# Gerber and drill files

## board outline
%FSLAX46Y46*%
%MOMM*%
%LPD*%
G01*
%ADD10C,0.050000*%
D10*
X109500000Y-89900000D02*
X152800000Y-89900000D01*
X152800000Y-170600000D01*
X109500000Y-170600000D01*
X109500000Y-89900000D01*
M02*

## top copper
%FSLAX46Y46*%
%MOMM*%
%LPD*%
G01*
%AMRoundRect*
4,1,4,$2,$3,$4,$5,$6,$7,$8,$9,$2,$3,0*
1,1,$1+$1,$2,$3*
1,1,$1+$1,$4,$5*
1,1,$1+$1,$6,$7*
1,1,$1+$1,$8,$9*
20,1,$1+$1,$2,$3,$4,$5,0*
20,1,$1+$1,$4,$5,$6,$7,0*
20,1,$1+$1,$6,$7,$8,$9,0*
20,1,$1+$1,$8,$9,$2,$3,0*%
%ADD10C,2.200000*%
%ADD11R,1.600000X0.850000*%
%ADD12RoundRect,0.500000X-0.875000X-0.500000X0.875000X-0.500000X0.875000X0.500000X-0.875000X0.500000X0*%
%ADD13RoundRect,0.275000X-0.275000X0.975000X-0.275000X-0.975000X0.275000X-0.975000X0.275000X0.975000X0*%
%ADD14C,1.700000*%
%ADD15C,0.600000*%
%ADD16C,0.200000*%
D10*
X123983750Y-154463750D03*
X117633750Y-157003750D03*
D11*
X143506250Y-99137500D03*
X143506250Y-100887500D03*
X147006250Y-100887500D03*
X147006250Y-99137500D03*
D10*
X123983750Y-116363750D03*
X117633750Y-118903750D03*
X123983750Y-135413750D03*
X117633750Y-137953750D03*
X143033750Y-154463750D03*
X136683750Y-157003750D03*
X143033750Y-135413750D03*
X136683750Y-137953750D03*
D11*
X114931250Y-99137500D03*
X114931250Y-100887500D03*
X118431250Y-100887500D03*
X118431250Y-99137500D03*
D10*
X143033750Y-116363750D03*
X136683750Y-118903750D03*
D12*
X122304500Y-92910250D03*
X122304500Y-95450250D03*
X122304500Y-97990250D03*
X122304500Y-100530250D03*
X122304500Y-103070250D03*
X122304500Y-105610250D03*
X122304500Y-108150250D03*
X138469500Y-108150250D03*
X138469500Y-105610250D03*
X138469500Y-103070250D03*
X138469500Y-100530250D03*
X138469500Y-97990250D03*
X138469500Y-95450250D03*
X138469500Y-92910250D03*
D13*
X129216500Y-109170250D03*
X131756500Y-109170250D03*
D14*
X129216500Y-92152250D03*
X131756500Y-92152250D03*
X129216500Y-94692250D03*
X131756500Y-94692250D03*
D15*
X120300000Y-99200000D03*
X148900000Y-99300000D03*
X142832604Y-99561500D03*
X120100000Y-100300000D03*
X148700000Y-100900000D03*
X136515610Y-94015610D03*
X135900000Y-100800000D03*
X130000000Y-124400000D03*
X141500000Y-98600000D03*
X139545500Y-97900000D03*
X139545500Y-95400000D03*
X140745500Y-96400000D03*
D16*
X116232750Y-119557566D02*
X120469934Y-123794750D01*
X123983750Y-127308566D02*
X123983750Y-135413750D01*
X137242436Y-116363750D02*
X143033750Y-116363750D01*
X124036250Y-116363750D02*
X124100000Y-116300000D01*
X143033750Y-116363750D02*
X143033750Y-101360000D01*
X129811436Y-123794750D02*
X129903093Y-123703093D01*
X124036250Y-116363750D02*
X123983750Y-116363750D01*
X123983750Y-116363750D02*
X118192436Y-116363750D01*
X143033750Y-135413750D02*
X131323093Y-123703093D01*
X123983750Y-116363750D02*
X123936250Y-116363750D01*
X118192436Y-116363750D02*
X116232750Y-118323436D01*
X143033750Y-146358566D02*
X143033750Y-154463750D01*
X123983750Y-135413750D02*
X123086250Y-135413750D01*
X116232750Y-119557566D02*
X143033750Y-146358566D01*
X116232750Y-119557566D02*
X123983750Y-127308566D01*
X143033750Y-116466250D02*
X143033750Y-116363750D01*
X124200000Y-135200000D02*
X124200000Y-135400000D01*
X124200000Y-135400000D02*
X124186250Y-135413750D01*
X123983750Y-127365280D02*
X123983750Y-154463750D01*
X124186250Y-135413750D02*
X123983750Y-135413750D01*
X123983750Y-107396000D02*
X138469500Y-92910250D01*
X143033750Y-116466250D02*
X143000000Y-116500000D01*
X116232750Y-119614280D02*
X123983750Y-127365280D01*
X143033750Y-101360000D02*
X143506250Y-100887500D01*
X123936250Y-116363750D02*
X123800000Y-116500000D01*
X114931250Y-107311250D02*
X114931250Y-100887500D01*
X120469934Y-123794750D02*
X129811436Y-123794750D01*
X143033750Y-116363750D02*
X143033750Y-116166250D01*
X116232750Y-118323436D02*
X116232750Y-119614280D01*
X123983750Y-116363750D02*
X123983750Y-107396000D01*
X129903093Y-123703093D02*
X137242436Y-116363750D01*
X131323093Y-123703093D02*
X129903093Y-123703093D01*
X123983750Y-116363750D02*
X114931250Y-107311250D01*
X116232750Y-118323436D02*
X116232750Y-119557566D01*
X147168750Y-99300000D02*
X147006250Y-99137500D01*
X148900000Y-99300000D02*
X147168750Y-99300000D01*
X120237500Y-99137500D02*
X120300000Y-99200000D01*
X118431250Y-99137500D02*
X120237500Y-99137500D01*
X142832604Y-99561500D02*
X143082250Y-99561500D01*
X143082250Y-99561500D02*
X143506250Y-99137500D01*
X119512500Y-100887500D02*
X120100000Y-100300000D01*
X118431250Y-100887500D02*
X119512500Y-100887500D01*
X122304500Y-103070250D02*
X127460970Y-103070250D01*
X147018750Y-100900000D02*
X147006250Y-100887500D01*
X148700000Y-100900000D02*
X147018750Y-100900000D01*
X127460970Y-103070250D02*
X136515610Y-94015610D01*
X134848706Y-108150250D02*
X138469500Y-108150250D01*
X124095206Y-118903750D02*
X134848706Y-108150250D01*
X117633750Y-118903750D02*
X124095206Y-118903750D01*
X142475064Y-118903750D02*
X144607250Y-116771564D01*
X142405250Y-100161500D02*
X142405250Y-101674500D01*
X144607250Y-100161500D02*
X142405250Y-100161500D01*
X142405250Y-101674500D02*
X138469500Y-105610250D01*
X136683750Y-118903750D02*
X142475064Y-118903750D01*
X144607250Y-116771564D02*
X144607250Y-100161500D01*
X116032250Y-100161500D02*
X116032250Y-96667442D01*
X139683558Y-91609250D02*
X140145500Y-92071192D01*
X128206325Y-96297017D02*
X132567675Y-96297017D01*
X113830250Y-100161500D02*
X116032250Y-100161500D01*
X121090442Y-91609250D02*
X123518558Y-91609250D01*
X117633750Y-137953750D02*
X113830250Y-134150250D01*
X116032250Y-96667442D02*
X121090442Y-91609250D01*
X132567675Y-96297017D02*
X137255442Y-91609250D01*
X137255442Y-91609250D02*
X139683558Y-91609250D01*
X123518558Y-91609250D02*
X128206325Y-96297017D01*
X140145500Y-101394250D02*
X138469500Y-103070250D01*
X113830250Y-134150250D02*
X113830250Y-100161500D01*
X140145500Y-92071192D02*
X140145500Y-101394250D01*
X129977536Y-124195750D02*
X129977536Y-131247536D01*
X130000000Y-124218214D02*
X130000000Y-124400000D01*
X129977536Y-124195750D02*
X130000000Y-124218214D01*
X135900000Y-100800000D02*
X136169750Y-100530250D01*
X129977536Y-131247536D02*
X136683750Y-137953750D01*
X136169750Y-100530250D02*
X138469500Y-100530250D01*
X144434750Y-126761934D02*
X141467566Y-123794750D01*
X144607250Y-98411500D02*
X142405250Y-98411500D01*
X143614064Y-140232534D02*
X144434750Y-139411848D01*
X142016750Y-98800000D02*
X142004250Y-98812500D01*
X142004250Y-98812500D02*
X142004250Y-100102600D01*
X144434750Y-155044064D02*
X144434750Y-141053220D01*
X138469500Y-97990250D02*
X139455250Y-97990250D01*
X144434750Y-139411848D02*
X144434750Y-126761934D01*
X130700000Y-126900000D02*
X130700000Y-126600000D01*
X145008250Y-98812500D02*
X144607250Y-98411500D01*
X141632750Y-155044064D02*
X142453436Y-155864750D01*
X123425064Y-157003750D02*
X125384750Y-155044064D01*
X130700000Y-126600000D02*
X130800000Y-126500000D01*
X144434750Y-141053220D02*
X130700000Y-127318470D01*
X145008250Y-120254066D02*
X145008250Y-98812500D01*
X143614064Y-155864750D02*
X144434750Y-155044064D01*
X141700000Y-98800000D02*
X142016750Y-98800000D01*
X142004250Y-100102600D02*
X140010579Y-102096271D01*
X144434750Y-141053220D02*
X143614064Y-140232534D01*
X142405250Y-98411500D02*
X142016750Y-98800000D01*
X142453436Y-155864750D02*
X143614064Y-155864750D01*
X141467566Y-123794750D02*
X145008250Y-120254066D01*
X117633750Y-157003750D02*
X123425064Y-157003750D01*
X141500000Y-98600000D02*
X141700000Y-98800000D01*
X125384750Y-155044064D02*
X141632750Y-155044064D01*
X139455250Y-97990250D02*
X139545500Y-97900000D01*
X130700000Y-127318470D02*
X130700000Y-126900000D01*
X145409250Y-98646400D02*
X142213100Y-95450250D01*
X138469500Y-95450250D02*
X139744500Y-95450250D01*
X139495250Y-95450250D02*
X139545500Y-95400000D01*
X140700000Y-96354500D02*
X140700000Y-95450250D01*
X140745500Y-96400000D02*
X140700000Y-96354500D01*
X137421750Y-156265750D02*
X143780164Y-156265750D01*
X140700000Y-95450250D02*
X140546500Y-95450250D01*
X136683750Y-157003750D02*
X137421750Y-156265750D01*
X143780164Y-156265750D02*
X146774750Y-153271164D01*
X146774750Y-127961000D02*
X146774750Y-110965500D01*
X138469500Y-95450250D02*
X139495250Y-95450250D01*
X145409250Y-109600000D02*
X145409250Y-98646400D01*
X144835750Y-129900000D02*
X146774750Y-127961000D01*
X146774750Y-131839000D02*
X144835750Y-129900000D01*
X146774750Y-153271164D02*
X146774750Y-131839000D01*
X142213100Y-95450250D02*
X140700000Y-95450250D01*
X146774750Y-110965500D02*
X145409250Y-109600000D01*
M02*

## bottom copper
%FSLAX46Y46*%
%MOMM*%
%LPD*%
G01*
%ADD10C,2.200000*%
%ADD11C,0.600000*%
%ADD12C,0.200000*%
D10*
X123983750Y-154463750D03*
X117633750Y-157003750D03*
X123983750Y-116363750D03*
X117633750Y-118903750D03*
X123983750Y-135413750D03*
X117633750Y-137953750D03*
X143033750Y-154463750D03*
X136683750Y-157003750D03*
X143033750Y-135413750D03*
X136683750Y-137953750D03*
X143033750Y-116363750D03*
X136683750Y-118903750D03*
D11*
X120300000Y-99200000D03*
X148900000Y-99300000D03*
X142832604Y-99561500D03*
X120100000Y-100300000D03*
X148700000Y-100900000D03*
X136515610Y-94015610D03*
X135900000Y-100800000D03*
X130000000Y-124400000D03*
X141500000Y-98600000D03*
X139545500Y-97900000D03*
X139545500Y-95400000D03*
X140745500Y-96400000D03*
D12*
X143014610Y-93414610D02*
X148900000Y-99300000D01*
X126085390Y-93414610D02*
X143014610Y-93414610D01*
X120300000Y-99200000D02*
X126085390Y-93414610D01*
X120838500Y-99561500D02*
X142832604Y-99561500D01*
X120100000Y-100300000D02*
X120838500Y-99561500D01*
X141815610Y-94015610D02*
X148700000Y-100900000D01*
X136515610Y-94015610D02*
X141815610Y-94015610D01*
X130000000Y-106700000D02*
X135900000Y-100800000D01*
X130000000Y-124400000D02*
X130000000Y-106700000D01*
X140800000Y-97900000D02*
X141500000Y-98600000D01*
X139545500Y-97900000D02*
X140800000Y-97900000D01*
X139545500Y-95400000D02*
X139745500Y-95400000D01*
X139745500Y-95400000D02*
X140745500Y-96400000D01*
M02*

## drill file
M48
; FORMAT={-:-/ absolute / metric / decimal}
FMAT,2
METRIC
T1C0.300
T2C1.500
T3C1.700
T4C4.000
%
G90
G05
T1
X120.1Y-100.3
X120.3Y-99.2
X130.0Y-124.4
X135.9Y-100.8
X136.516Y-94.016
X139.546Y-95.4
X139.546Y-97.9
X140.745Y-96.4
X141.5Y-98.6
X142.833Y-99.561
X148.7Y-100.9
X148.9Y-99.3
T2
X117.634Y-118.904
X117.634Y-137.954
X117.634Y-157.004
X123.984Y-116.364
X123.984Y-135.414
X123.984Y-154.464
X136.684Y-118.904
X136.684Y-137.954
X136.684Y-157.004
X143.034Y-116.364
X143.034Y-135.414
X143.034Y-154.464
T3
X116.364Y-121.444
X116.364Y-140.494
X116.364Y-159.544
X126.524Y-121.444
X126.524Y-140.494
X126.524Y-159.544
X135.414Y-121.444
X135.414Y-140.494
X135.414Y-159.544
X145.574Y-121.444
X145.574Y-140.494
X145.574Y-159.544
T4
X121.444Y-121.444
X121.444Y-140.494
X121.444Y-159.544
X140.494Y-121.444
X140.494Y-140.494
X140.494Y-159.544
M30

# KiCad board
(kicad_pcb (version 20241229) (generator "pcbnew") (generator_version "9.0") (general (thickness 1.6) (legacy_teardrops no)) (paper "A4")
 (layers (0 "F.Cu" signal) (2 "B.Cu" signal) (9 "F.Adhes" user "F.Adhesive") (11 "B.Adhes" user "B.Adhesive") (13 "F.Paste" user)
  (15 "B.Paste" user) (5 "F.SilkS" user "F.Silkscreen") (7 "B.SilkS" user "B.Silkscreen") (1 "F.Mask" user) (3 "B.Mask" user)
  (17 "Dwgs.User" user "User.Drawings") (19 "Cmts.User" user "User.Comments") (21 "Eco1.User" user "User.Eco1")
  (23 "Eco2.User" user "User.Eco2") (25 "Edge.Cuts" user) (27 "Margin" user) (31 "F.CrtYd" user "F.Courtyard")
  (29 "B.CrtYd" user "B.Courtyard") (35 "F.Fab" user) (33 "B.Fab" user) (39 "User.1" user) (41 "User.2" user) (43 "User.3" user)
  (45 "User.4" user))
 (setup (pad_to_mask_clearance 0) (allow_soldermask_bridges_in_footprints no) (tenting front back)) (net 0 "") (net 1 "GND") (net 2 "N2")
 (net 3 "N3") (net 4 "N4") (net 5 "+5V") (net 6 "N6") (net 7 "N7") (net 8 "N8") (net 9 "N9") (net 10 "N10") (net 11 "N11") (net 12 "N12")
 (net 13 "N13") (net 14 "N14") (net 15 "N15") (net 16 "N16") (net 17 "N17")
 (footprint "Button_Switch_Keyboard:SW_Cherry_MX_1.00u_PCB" (layer "F.Cu") (at 123.98375 154.46375)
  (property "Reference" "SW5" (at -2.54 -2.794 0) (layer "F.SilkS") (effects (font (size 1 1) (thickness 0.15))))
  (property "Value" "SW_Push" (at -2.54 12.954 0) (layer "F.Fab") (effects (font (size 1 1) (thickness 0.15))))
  (pad "" np_thru_hole circle (at -7.62 5.08) (size 1.7 1.7) (drill 1.7) (layers "*.Cu" "*.Mask"))
  (pad "" np_thru_hole circle (at -2.54 5.08) (size 4 4) (drill 4) (layers "*.Cu" "*.Mask"))
  (pad "" np_thru_hole circle (at 2.54 5.08) (size 1.7 1.7) (drill 1.7) (layers "*.Cu" "*.Mask"))
  (pad "1" thru_hole circle (at 0 0) (size 2.2 2.2) (drill 1.5) (layers "*.Cu" "*.Mask") (remove_unused_layers no) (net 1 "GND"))
  (pad "2" thru_hole circle (at -6.35 2.54) (size 2.2 2.2) (drill 1.5) (layers "*.Cu" "*.Mask") (remove_unused_layers no) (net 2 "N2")))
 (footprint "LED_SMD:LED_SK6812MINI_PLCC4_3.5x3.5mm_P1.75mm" (layer "F.Cu") (at 145.25625 100.0125)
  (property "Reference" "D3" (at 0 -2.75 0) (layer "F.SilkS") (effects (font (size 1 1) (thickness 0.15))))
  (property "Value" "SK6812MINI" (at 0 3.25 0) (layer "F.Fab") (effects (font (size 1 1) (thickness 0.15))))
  (pad "1" smd rect (at -1.75 -0.875) (size 1.6 0.85) (layers "F.Cu" "F.Mask" "F.Paste") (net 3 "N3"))
  (pad "2" smd rect (at -1.75 0.875) (size 1.6 0.85) (layers "F.Cu" "F.Mask" "F.Paste") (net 1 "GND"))
  (pad "3" smd rect (at 1.75 0.875) (size 1.6 0.85) (layers "F.Cu" "F.Mask" "F.Paste") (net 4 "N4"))
  (pad "4" smd rect (at 1.75 -0.875) (size 1.6 0.85) (layers "F.Cu" "F.Mask" "F.Paste") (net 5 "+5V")))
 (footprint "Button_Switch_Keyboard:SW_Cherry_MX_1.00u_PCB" (layer "F.Cu") (at 123.98375 116.36375)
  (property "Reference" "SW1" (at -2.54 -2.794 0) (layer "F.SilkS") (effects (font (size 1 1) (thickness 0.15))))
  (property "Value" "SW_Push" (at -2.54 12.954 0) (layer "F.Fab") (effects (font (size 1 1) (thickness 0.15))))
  (pad "" np_thru_hole circle (at -7.62 5.08) (size 1.7 1.7) (drill 1.7) (layers "*.Cu" "*.Mask"))
  (pad "" np_thru_hole circle (at -2.54 5.08) (size 4 4) (drill 4) (layers "*.Cu" "*.Mask"))
  (pad "" np_thru_hole circle (at 2.54 5.08) (size 1.7 1.7) (drill 1.7) (layers "*.Cu" "*.Mask"))
  (pad "1" thru_hole circle (at 0 0) (size 2.2 2.2) (drill 1.5) (layers "*.Cu" "*.Mask") (remove_unused_layers no) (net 1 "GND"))
  (pad "2" thru_hole circle (at -6.35 2.54) (size 2.2 2.2) (drill 1.5) (layers "*.Cu" "*.Mask") (remove_unused_layers no) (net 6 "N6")))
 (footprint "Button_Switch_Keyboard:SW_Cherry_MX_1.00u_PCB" (layer "F.Cu") (at 123.98375 135.41375)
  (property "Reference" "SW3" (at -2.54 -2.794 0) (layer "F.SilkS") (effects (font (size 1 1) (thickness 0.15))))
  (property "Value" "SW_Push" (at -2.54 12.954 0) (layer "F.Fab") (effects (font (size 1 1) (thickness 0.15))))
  (pad "" np_thru_hole circle (at -7.62 5.08) (size 1.7 1.7) (drill 1.7) (layers "*.Cu" "*.Mask"))
  (pad "" np_thru_hole circle (at -2.54 5.08) (size 4 4) (drill 4) (layers "*.Cu" "*.Mask"))
  (pad "" np_thru_hole circle (at 2.54 5.08) (size 1.7 1.7) (drill 1.7) (layers "*.Cu" "*.Mask"))
  (pad "1" thru_hole circle (at 0 0) (size 2.2 2.2) (drill 1.5) (layers "*.Cu" "*.Mask") (remove_unused_layers no) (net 1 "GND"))
  (pad "2" thru_hole circle (at -6.35 2.54) (size 2.2 2.2) (drill 1.5) (layers "*.Cu" "*.Mask") (remove_unused_layers no) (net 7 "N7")))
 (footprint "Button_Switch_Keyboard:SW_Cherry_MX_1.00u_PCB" (layer "F.Cu") (at 143.03375 154.46375)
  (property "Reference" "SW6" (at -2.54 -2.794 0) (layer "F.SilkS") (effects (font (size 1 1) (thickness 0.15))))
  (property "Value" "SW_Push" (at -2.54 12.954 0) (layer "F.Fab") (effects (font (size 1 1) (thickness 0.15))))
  (pad "" np_thru_hole circle (at -7.62 5.08) (size 1.7 1.7) (drill 1.7) (layers "*.Cu" "*.Mask"))
  (pad "" np_thru_hole circle (at -2.54 5.08) (size 4 4) (drill 4) (layers "*.Cu" "*.Mask"))
  (pad "" np_thru_hole circle (at 2.54 5.08) (size 1.7 1.7) (drill 1.7) (layers "*.Cu" "*.Mask"))
  (pad "1" thru_hole circle (at 0 0) (size 2.2 2.2) (drill 1.5) (layers "*.Cu" "*.Mask") (remove_unused_layers no) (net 1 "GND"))
  (pad "2" thru_hole circle (at -6.35 2.54) (size 2.2 2.2) (drill 1.5) (layers "*.Cu" "*.Mask") (remove_unused_layers no) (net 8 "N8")))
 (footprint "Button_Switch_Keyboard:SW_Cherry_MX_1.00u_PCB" (layer "F.Cu") (at 143.03375 135.41375)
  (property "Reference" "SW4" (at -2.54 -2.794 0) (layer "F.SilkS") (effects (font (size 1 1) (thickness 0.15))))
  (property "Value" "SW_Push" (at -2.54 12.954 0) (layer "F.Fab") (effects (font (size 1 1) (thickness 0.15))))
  (pad "" np_thru_hole circle (at -7.62 5.08) (size 1.7 1.7) (drill 1.7) (layers "*.Cu" "*.Mask"))
  (pad "" np_thru_hole circle (at -2.54 5.08) (size 4 4) (drill 4) (layers "*.Cu" "*.Mask"))
  (pad "" np_thru_hole circle (at 2.54 5.08) (size 1.7 1.7) (drill 1.7) (layers "*.Cu" "*.Mask"))
  (pad "1" thru_hole circle (at 0 0) (size 2.2 2.2) (drill 1.5) (layers "*.Cu" "*.Mask") (remove_unused_layers no) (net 1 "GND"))
  (pad "2" thru_hole circle (at -6.35 2.54) (size 2.2 2.2) (drill 1.5) (layers "*.Cu" "*.Mask") (remove_unused_layers no) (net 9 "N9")))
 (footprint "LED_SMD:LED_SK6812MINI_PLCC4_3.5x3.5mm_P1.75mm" (layer "F.Cu") (at 116.68125 100.0125)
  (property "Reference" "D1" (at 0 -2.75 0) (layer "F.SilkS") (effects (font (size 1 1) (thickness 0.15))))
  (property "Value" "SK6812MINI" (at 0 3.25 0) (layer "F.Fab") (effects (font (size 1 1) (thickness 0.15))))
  (pad "1" smd rect (at -1.75 -0.875) (size 1.6 0.85) (layers "F.Cu" "F.Mask" "F.Paste") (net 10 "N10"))
  (pad "2" smd rect (at -1.75 0.875) (size 1.6 0.85) (layers "F.Cu" "F.Mask" "F.Paste") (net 1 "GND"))
  (pad "3" smd rect (at 1.75 0.875) (size 1.6 0.85) (layers "F.Cu" "F.Mask" "F.Paste") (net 3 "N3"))
  (pad "4" smd rect (at 1.75 -0.875) (size 1.6 0.85) (layers "F.Cu" "F.Mask" "F.Paste") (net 5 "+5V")))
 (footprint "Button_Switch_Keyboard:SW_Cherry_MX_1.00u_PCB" (layer "F.Cu") (at 143.03375 116.36375)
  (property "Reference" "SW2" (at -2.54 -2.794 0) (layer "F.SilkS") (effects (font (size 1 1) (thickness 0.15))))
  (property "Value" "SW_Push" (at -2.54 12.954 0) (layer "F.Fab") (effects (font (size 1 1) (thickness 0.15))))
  (pad "" np_thru_hole circle (at -7.62 5.08) (size 1.7 1.7) (drill 1.7) (layers "*.Cu" "*.Mask"))
  (pad "" np_thru_hole circle (at -2.54 5.08) (size 4 4) (drill 4) (layers "*.Cu" "*.Mask"))
  (pad "" np_thru_hole circle (at 2.54 5.08) (size 1.7 1.7) (drill 1.7) (layers "*.Cu" "*.Mask"))
  (pad "1" thru_hole circle (at 0 0) (size 2.2 2.2) (drill 1.5) (layers "*.Cu" "*.Mask") (remove_unused_layers no) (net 1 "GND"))
  (pad "2" thru_hole circle (at -6.35 2.54) (size 2.2 2.2) (drill 1.5) (layers "*.Cu" "*.Mask") (remove_unused_layers no) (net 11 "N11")))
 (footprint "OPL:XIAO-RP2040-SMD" (layer "F.Cu") (at 130.3045 100.53025)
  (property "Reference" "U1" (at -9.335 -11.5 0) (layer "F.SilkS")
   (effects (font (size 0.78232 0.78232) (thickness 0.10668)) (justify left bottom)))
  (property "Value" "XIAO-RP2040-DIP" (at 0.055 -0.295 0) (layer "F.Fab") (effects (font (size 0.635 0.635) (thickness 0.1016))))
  (pad "1" smd roundrect (at -8 -7.62) (size 2.75 2) (layers "F.Cu" "F.Mask" "F.Paste") (roundrect_rratio 0.25) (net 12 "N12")
   (solder_mask_margin 0.0508) (thermal_bridge_angle 45))
  (pad "2" smd roundrect (at -8 -5.08) (size 2.75 2) (layers "F.Cu" "F.Mask" "F.Paste") (roundrect_rratio 0.25) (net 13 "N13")
   (solder_mask_margin 0.0508) (thermal_bridge_angle 45))
  (pad "3" smd roundrect (at -8 -2.54) (size 2.75 2) (layers "F.Cu" "F.Mask" "F.Paste") (roundrect_rratio 0.25) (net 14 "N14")
   (solder_mask_margin 0.0508) (thermal_bridge_angle 45))
  (pad "4" smd roundrect (at -8 0) (size 2.75 2) (layers "F.Cu" "F.Mask" "F.Paste") (roundrect_rratio 0.25) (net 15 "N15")
   (solder_mask_margin 0.0508) (thermal_bridge_angle 45))
  (pad "5" smd roundrect (at -8 2.54) (size 2.75 2) (layers "F.Cu" "F.Mask" "F.Paste") (roundrect_rratio 0.25) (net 4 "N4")
   (solder_mask_margin 0.0508) (thermal_bridge_angle 45))
  (pad "6" smd roundrect (at -8 5.08) (size 2.75 2) (layers "F.Cu" "F.Mask" "F.Paste") (roundrect_rratio 0.25) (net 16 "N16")
   (solder_mask_margin 0.0508) (thermal_bridge_angle 45))
  (pad "7" smd roundrect (at -8 7.62) (size 2.75 2) (layers "F.Cu" "F.Mask" "F.Paste") (roundrect_rratio 0.25) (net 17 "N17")
   (solder_mask_margin 0.0508) (thermal_bridge_angle 45))
  (pad "8" smd roundrect (at 8.165 7.62) (size 2.75 2) (layers "F.Cu" "F.Mask" "F.Paste") (roundrect_rratio 0.25) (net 6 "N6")
   (solder_mask_margin 0.0508) (thermal_bridge_angle 45))
  (pad "9" smd roundrect (at 8.165 5.08) (size 2.75 2) (layers "F.Cu" "F.Mask" "F.Paste") (roundrect_rratio 0.25) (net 11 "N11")
   (solder_mask_margin 0.0508) (thermal_bridge_angle 45))
  (pad "10" smd roundrect (at 8.165 2.54) (size 2.75 2) (layers "F.Cu" "F.Mask" "F.Paste") (roundrect_rratio 0.25) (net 7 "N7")
   (solder_mask_margin 0.0508) (thermal_bridge_angle 45))
  (pad "11" smd roundrect (at 8.165 0) (size 2.75 2) (layers "F.Cu" "F.Mask" "F.Paste") (roundrect_rratio 0.25) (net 9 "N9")
   (solder_mask_margin 0.0508) (thermal_bridge_angle 45))
  (pad "12" smd roundrect (at 8.165 -2.54) (size 2.75 2) (layers "F.Cu" "F.Mask" "F.Paste") (roundrect_rratio 0.25) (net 2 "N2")
   (solder_mask_margin 0.0508) (thermal_bridge_angle 45))
  (pad "13" smd roundrect (at 8.165 -5.08) (size 2.75 2) (layers "F.Cu" "F.Mask" "F.Paste") (roundrect_rratio 0.25) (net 8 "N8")
   (solder_mask_margin 0.0508) (thermal_bridge_angle 45))
  (pad "14" smd roundrect (at 8.165 -7.62) (size 2.75 2) (layers "F.Cu" "F.Mask" "F.Paste") (roundrect_rratio 0.25) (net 1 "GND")
   (solder_mask_margin 0.0508) (thermal_bridge_angle 45))
  (pad "15" smd roundrect (at -1.088 8.64 270) (size 2.5 1.1) (layers "F.Cu" "F.Mask" "F.Paste") (roundrect_rratio 0.25)
   (thermal_bridge_angle 45))
  (pad "16" smd roundrect (at 1.452 8.64 270) (size 2.5 1.1) (layers "F.Cu" "F.Mask" "F.Paste") (roundrect_rratio 0.25)
   (thermal_bridge_angle 45))
  (pad "17" smd circle (at -1.088 -8.378) (size 1.7 1.7) (layers "F.Cu" "F.Mask" "F.Paste"))
  (pad "18" smd circle (at 1.452 -8.378) (size 1.7 1.7) (layers "F.Cu" "F.Mask" "F.Paste"))
  (pad "19" smd circle (at -1.088 -5.838) (size 1.7 1.7) (layers "F.Cu" "F.Mask" "F.Paste"))
  (pad "20" smd circle (at 1.452 -5.838) (size 1.7 1.7) (layers "F.Cu" "F.Mask" "F.Paste")))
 (gr_rect (start 109.5 89.9) (end 152.8 170.6) (stroke (width 0.05) (type default)) (fill no) (layer "Edge.Cuts"))
 (segment (start 116.23275 119.557566) (end 120.469934 123.79475) (width 0.2) (layer "F.Cu") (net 1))
 (segment (start 123.98375 127.308566) (end 123.98375 135.41375) (width 0.2) (layer "F.Cu") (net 1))
 (segment (start 137.242436 116.36375) (end 143.03375 116.36375) (width 0.2) (layer "F.Cu") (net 1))
 (segment (start 124.03625 116.36375) (end 124.1 116.3) (width 0.2) (layer "F.Cu") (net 1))
 (segment (start 143.03375 116.36375) (end 143.03375 101.36) (width 0.2) (layer "F.Cu") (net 1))
 (segment (start 129.811436 123.79475) (end 129.903093 123.703093) (width 0.2) (layer "F.Cu") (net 1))
 (segment (start 124.03625 116.36375) (end 123.98375 116.36375) (width 0.2) (layer "F.Cu") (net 1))
 (segment (start 123.98375 116.36375) (end 118.192436 116.36375) (width 0.2) (layer "F.Cu") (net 1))
 (segment (start 143.03375 135.41375) (end 131.323093 123.703093) (width 0.2) (layer "F.Cu") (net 1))
 (segment (start 123.98375 116.36375) (end 123.93625 116.36375) (width 0.2) (layer "F.Cu") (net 1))
 (segment (start 118.192436 116.36375) (end 116.23275 118.323436) (width 0.2) (layer "F.Cu") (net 1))
 (segment (start 143.03375 146.358566) (end 143.03375 154.46375) (width 0.2) (layer "F.Cu") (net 1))
 (segment (start 123.98375 135.41375) (end 123.08625 135.41375) (width 0.2) (layer "F.Cu") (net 1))
 (segment (start 116.23275 119.557566) (end 143.03375 146.358566) (width 0.2) (layer "F.Cu") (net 1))
 (segment (start 116.23275 119.557566) (end 123.98375 127.308566) (width 0.2) (layer "F.Cu") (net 1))
 (segment (start 143.03375 116.46625) (end 143.03375 116.36375) (width 0.2) (layer "F.Cu") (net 1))
 (segment (start 124.2 135.2) (end 124.2 135.4) (width 0.2) (layer "F.Cu") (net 1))
 (segment (start 124.2 135.4) (end 124.18625 135.41375) (width 0.2) (layer "F.Cu") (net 1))
 (segment (start 123.98375 127.36528) (end 123.98375 154.46375) (width 0.2) (layer "F.Cu") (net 1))
 (segment (start 124.18625 135.41375) (end 123.98375 135.41375) (width 0.2) (layer "F.Cu") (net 1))
 (segment (start 123.98375 107.396) (end 138.4695 92.91025) (width 0.2) (layer "F.Cu") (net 1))
 (segment (start 143.03375 116.46625) (end 143 116.5) (width 0.2) (layer "F.Cu") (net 1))
 (segment (start 116.23275 119.61428) (end 123.98375 127.36528) (width 0.2) (layer "F.Cu") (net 1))
 (segment (start 143.03375 101.36) (end 143.50625 100.8875) (width 0.2) (layer "F.Cu") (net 1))
 (segment (start 123.93625 116.36375) (end 123.8 116.5) (width 0.2) (layer "F.Cu") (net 1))
 (segment (start 114.93125 107.31125) (end 114.93125 100.8875) (width 0.2) (layer "F.Cu") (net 1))
 (segment (start 120.469934 123.79475) (end 129.811436 123.79475) (width 0.2) (layer "F.Cu") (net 1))
 (segment (start 143.03375 116.36375) (end 143.03375 116.16625) (width 0.2) (layer "F.Cu") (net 1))
 (segment (start 116.23275 118.323436) (end 116.23275 119.61428) (width 0.2) (layer "F.Cu") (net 1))
 (segment (start 123.98375 116.36375) (end 123.98375 107.396) (width 0.2) (layer "F.Cu") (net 1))
 (segment (start 129.903093 123.703093) (end 137.242436 116.36375) (width 0.2) (layer "F.Cu") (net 1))
 (segment (start 131.323093 123.703093) (end 129.903093 123.703093) (width 0.2) (layer "F.Cu") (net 1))
 (segment (start 123.98375 116.36375) (end 114.93125 107.31125) (width 0.2) (layer "F.Cu") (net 1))
 (segment (start 116.23275 118.323436) (end 116.23275 119.557566) (width 0.2) (layer "F.Cu") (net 1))
 (segment (start 147.16875 99.3) (end 147.00625 99.1375) (width 0.2) (layer "F.Cu") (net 5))
 (segment (start 148.9 99.3) (end 147.16875 99.3) (width 0.2) (layer "F.Cu") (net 5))
 (segment (start 120.2375 99.1375) (end 120.3 99.2) (width 0.2) (layer "F.Cu") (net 5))
 (segment (start 118.43125 99.1375) (end 120.2375 99.1375) (width 0.2) (layer "F.Cu") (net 5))
 (via (at 120.3 99.2) (size 0.6) (drill 0.3) (layers "F.Cu" "B.Cu") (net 5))
 (via (at 148.9 99.3) (size 0.6) (drill 0.3) (layers "F.Cu" "B.Cu") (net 5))
 (segment (start 143.01461 93.41461) (end 148.9 99.3) (width 0.2) (layer "B.Cu") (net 5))
 (segment (start 126.08539 93.41461) (end 143.01461 93.41461) (width 0.2) (layer "B.Cu") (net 5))
 (segment (start 120.3 99.2) (end 126.08539 93.41461) (width 0.2) (layer "B.Cu") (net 5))
 (segment (start 142.832604 99.5615) (end 143.08225 99.5615) (width 0.2) (layer "F.Cu") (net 3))
 (segment (start 143.08225 99.5615) (end 143.50625 99.1375) (width 0.2) (layer "F.Cu") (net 3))
 (segment (start 119.5125 100.8875) (end 120.1 100.3) (width 0.2) (layer "F.Cu") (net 3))
 (segment (start 118.43125 100.8875) (end 119.5125 100.8875) (width 0.2) (layer "F.Cu") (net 3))
 (via (at 142.832604 99.5615) (size 0.6) (drill 0.3) (layers "F.Cu" "B.Cu") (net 3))
 (via (at 120.1 100.3) (size 0.6) (drill 0.3) (layers "F.Cu" "B.Cu") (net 3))
 (segment (start 120.8385 99.5615) (end 142.832604 99.5615) (width 0.2) (layer "B.Cu") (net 3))
 (segment (start 120.1 100.3) (end 120.8385 99.5615) (width 0.2) (layer "B.Cu") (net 3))
 (segment (start 122.3045 103.07025) (end 127.46097 103.07025) (width 0.2) (layer "F.Cu") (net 4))
 (segment (start 147.01875 100.9) (end 147.00625 100.8875) (width 0.2) (layer "F.Cu") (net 4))
 (segment (start 148.7 100.9) (end 147.01875 100.9) (width 0.2) (layer "F.Cu") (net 4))
 (segment (start 127.46097 103.07025) (end 136.51561 94.01561) (width 0.2) (layer "F.Cu") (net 4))
 (via (at 148.7 100.9) (size 0.6) (drill 0.3) (layers "F.Cu" "B.Cu") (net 4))
 (via (at 136.51561 94.01561) (size 0.6) (drill 0.3) (layers "F.Cu" "B.Cu") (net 4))
 (segment (start 141.81561 94.01561) (end 148.7 100.9) (width 0.2) (layer "B.Cu") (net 4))
 (segment (start 136.51561 94.01561) (end 141.81561 94.01561) (width 0.2) (layer "B.Cu") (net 4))
 (segment (start 134.848706 108.15025) (end 138.4695 108.15025) (width 0.2) (layer "F.Cu") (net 6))
 (segment (start 124.095206 118.90375) (end 134.848706 108.15025) (width 0.2) (layer "F.Cu") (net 6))
 (segment (start 117.63375 118.90375) (end 124.095206 118.90375) (width 0.2) (layer "F.Cu") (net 6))
 (segment (start 142.475064 118.90375) (end 144.60725 116.771564) (width 0.2) (layer "F.Cu") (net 11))
 (segment (start 142.40525 100.1615) (end 142.40525 101.6745) (width 0.2) (layer "F.Cu") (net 11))
 (segment (start 144.60725 100.1615) (end 142.40525 100.1615) (width 0.2) (layer "F.Cu") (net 11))
 (segment (start 142.40525 101.6745) (end 138.4695 105.61025) (width 0.2) (layer "F.Cu") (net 11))
 (segment (start 136.68375 118.90375) (end 142.475064 118.90375) (width 0.2) (layer "F.Cu") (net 11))
 (segment (start 144.60725 116.771564) (end 144.60725 100.1615) (width 0.2) (layer "F.Cu") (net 11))
 (segment (start 116.03225 100.1615) (end 116.03225 96.667442) (width 0.2) (layer "F.Cu") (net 7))
 (segment (start 139.683558 91.60925) (end 140.1455 92.071192) (width 0.2) (layer "F.Cu") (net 7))
 (segment (start 128.206325 96.297017) (end 132.567675 96.297017) (width 0.2) (layer "F.Cu") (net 7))
 (segment (start 113.83025 100.1615) (end 116.03225 100.1615) (width 0.2) (layer "F.Cu") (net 7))
 (segment (start 121.090442 91.60925) (end 123.518558 91.60925) (width 0.2) (layer "F.Cu") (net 7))
 (segment (start 117.63375 137.95375) (end 113.83025 134.15025) (width 0.2) (layer "F.Cu") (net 7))
 (segment (start 116.03225 96.667442) (end 121.090442 91.60925) (width 0.2) (layer "F.Cu") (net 7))
 (segment (start 132.567675 96.297017) (end 137.255442 91.60925) (width 0.2) (layer "F.Cu") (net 7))
 (segment (start 137.255442 91.60925) (end 139.683558 91.60925) (width 0.2) (layer "F.Cu") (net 7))
 (segment (start 123.518558 91.60925) (end 128.206325 96.297017) (width 0.2) (layer "F.Cu") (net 7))
 (segment (start 140.1455 101.39425) (end 138.4695 103.07025) (width 0.2) (layer "F.Cu") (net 7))
 (segment (start 113.83025 134.15025) (end 113.83025 100.1615) (width 0.2) (layer "F.Cu") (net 7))
 (segment (start 140.1455 92.071192) (end 140.1455 101.39425) (width 0.2) (layer "F.Cu") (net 7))
 (segment (start 129.977536 124.19575) (end 129.977536 131.247536) (width 0.2) (layer "F.Cu") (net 9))
 (segment (start 130 124.218214) (end 130 124.4) (width 0.2) (layer "F.Cu") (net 9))
 (segment (start 129.977536 124.19575) (end 130 124.218214) (width 0.2) (layer "F.Cu") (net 9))
 (segment (start 135.9 100.8) (end 136.16975 100.53025) (width 0.2) (layer "F.Cu") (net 9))
 (segment (start 129.977536 131.247536) (end 136.68375 137.95375) (width 0.2) (layer "F.Cu") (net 9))
 (segment (start 136.16975 100.53025) (end 138.4695 100.53025) (width 0.2) (layer "F.Cu") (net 9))
 (via (at 135.9 100.8) (size 0.6) (drill 0.3) (layers "F.Cu" "B.Cu") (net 9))
 (via (at 130 124.4) (size 0.6) (drill 0.3) (layers "F.Cu" "B.Cu") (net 9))
 (segment (start 130 106.7) (end 135.9 100.8) (width 0.2) (layer "B.Cu") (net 9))
 (segment (start 130 124.4) (end 130 106.7) (width 0.2) (layer "B.Cu") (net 9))
 (segment (start 144.43475 126.761934) (end 141.467566 123.79475) (width 0.2) (layer "F.Cu") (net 2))
 (segment (start 144.60725 98.4115) (end 142.40525 98.4115) (width 0.2) (layer "F.Cu") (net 2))
 (segment (start 143.614064 140.232534) (end 144.43475 139.411848) (width 0.2) (layer "F.Cu") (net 2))
 (segment (start 142.01675 98.8) (end 142.00425 98.8125) (width 0.2) (layer "F.Cu") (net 2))
 (segment (start 142.00425 98.8125) (end 142.00425 100.1026) (width 0.2) (layer "F.Cu") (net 2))
 (segment (start 144.43475 155.044064) (end 144.43475 141.05322) (width 0.2) (layer "F.Cu") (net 2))
 (segment (start 138.4695 97.99025) (end 139.45525 97.99025) (width 0.2) (layer "F.Cu") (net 2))
 (segment (start 144.43475 139.411848) (end 144.43475 126.761934) (width 0.2) (layer "F.Cu") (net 2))
 (segment (start 130.7 126.9) (end 130.7 126.6) (width 0.2) (layer "F.Cu") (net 2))
 (segment (start 145.00825 98.8125) (end 144.60725 98.4115) (width 0.2) (layer "F.Cu") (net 2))
 (segment (start 141.63275 155.044064) (end 142.453436 155.86475) (width 0.2) (layer "F.Cu") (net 2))
 (segment (start 123.425064 157.00375) (end 125.38475 155.044064) (width 0.2) (layer "F.Cu") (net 2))
 (segment (start 130.7 126.6) (end 130.8 126.5) (width 0.2) (layer "F.Cu") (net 2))
 (segment (start 144.43475 141.05322) (end 130.7 127.31847) (width 0.2) (layer "F.Cu") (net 2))
 (segment (start 145.00825 120.254066) (end 145.00825 98.8125) (width 0.2) (layer "F.Cu") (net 2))
 (segment (start 143.614064 155.86475) (end 144.43475 155.044064) (width 0.2) (layer "F.Cu") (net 2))
 (segment (start 141.7 98.8) (end 142.01675 98.8) (width 0.2) (layer "F.Cu") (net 2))
 (segment (start 142.00425 100.1026) (end 140.010579 102.096271) (width 0.2) (layer "F.Cu") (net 2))
 (segment (start 144.43475 141.05322) (end 143.614064 140.232534) (width 0.2) (layer "F.Cu") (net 2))
 (segment (start 142.40525 98.4115) (end 142.01675 98.8) (width 0.2) (layer "F.Cu") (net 2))
 (segment (start 142.453436 155.86475) (end 143.614064 155.86475) (width 0.2) (layer "F.Cu") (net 2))
 (segment (start 141.467566 123.79475) (end 145.00825 120.254066) (width 0.2) (layer "F.Cu") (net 2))
 (segment (start 117.63375 157.00375) (end 123.425064 157.00375) (width 0.2) (layer "F.Cu") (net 2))
 (segment (start 141.5 98.6) (end 141.7 98.8) (width 0.2) (layer "F.Cu") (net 2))
 (segment (start 125.38475 155.044064) (end 141.63275 155.044064) (width 0.2) (layer "F.Cu") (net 2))
 (segment (start 139.45525 97.99025) (end 139.5455 97.9) (width 0.2) (layer "F.Cu") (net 2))
 (segment (start 130.7 127.31847) (end 130.7 126.9) (width 0.2) (layer "F.Cu") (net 2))
 (via (at 141.5 98.6) (size 0.6) (drill 0.3) (layers "F.Cu" "B.Cu") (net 2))
 (via (at 139.5455 97.9) (size 0.6) (drill 0.3) (layers "F.Cu" "B.Cu") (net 2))
 (segment (start 140.8 97.9) (end 141.5 98.6) (width 0.2) (layer "B.Cu") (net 2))
 (segment (start 139.5455 97.9) (end 140.8 97.9) (width 0.2) (layer "B.Cu") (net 2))
 (segment (start 145.40925 98.6464) (end 142.2131 95.45025) (width 0.2) (layer "F.Cu") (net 8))
 (segment (start 138.4695 95.45025) (end 139.7445 95.45025) (width 0.2) (layer "F.Cu") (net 8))
 (segment (start 139.49525 95.45025) (end 139.5455 95.4) (width 0.2) (layer "F.Cu") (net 8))
 (segment (start 140.7 96.3545) (end 140.7 95.45025) (width 0.2) (layer "F.Cu") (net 8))
 (segment (start 140.7455 96.4) (end 140.7 96.3545) (width 0.2) (layer "F.Cu") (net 8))
 (segment (start 137.42175 156.26575) (end 143.780164 156.26575) (width 0.2) (layer "F.Cu") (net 8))
 (segment (start 140.7 95.45025) (end 140.5465 95.45025) (width 0.2) (layer "F.Cu") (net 8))
 (segment (start 136.68375 157.00375) (end 137.42175 156.26575) (width 0.2) (layer "F.Cu") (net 8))
 (segment (start 143.780164 156.26575) (end 146.77475 153.271164) (width 0.2) (layer "F.Cu") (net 8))
 (segment (start 146.77475 127.961) (end 146.77475 110.9655) (width 0.2) (layer "F.Cu") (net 8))
 (segment (start 138.4695 95.45025) (end 139.49525 95.45025) (width 0.2) (layer "F.Cu") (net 8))
 (segment (start 145.40925 109.6) (end 145.40925 98.6464) (width 0.2) (layer "F.Cu") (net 8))
 (segment (start 144.83575 129.9) (end 146.77475 127.961) (width 0.2) (layer "F.Cu") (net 8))
 (segment (start 146.77475 131.839) (end 144.83575 129.9) (width 0.2) (layer "F.Cu") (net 8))
 (segment (start 146.77475 153.271164) (end 146.77475 131.839) (width 0.2) (layer "F.Cu") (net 8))
 (segment (start 142.2131 95.45025) (end 140.7 95.45025) (width 0.2) (layer "F.Cu") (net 8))
 (segment (start 146.77475 110.9655) (end 145.40925 109.6) (width 0.2) (layer "F.Cu") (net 8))
 (via (at 139.5455 95.4) (size 0.6) (drill 0.3) (layers "F.Cu" "B.Cu") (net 8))
 (via (at 140.7455 96.4) (size 0.6) (drill 0.3) (layers "F.Cu" "B.Cu") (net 8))
 (segment (start 139.5455 95.4) (end 139.7455 95.4) (width 0.2) (layer "B.Cu") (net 8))
 (segment (start 139.7455 95.4) (end 140.7455 96.4) (width 0.2) (layer "B.Cu") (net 8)))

